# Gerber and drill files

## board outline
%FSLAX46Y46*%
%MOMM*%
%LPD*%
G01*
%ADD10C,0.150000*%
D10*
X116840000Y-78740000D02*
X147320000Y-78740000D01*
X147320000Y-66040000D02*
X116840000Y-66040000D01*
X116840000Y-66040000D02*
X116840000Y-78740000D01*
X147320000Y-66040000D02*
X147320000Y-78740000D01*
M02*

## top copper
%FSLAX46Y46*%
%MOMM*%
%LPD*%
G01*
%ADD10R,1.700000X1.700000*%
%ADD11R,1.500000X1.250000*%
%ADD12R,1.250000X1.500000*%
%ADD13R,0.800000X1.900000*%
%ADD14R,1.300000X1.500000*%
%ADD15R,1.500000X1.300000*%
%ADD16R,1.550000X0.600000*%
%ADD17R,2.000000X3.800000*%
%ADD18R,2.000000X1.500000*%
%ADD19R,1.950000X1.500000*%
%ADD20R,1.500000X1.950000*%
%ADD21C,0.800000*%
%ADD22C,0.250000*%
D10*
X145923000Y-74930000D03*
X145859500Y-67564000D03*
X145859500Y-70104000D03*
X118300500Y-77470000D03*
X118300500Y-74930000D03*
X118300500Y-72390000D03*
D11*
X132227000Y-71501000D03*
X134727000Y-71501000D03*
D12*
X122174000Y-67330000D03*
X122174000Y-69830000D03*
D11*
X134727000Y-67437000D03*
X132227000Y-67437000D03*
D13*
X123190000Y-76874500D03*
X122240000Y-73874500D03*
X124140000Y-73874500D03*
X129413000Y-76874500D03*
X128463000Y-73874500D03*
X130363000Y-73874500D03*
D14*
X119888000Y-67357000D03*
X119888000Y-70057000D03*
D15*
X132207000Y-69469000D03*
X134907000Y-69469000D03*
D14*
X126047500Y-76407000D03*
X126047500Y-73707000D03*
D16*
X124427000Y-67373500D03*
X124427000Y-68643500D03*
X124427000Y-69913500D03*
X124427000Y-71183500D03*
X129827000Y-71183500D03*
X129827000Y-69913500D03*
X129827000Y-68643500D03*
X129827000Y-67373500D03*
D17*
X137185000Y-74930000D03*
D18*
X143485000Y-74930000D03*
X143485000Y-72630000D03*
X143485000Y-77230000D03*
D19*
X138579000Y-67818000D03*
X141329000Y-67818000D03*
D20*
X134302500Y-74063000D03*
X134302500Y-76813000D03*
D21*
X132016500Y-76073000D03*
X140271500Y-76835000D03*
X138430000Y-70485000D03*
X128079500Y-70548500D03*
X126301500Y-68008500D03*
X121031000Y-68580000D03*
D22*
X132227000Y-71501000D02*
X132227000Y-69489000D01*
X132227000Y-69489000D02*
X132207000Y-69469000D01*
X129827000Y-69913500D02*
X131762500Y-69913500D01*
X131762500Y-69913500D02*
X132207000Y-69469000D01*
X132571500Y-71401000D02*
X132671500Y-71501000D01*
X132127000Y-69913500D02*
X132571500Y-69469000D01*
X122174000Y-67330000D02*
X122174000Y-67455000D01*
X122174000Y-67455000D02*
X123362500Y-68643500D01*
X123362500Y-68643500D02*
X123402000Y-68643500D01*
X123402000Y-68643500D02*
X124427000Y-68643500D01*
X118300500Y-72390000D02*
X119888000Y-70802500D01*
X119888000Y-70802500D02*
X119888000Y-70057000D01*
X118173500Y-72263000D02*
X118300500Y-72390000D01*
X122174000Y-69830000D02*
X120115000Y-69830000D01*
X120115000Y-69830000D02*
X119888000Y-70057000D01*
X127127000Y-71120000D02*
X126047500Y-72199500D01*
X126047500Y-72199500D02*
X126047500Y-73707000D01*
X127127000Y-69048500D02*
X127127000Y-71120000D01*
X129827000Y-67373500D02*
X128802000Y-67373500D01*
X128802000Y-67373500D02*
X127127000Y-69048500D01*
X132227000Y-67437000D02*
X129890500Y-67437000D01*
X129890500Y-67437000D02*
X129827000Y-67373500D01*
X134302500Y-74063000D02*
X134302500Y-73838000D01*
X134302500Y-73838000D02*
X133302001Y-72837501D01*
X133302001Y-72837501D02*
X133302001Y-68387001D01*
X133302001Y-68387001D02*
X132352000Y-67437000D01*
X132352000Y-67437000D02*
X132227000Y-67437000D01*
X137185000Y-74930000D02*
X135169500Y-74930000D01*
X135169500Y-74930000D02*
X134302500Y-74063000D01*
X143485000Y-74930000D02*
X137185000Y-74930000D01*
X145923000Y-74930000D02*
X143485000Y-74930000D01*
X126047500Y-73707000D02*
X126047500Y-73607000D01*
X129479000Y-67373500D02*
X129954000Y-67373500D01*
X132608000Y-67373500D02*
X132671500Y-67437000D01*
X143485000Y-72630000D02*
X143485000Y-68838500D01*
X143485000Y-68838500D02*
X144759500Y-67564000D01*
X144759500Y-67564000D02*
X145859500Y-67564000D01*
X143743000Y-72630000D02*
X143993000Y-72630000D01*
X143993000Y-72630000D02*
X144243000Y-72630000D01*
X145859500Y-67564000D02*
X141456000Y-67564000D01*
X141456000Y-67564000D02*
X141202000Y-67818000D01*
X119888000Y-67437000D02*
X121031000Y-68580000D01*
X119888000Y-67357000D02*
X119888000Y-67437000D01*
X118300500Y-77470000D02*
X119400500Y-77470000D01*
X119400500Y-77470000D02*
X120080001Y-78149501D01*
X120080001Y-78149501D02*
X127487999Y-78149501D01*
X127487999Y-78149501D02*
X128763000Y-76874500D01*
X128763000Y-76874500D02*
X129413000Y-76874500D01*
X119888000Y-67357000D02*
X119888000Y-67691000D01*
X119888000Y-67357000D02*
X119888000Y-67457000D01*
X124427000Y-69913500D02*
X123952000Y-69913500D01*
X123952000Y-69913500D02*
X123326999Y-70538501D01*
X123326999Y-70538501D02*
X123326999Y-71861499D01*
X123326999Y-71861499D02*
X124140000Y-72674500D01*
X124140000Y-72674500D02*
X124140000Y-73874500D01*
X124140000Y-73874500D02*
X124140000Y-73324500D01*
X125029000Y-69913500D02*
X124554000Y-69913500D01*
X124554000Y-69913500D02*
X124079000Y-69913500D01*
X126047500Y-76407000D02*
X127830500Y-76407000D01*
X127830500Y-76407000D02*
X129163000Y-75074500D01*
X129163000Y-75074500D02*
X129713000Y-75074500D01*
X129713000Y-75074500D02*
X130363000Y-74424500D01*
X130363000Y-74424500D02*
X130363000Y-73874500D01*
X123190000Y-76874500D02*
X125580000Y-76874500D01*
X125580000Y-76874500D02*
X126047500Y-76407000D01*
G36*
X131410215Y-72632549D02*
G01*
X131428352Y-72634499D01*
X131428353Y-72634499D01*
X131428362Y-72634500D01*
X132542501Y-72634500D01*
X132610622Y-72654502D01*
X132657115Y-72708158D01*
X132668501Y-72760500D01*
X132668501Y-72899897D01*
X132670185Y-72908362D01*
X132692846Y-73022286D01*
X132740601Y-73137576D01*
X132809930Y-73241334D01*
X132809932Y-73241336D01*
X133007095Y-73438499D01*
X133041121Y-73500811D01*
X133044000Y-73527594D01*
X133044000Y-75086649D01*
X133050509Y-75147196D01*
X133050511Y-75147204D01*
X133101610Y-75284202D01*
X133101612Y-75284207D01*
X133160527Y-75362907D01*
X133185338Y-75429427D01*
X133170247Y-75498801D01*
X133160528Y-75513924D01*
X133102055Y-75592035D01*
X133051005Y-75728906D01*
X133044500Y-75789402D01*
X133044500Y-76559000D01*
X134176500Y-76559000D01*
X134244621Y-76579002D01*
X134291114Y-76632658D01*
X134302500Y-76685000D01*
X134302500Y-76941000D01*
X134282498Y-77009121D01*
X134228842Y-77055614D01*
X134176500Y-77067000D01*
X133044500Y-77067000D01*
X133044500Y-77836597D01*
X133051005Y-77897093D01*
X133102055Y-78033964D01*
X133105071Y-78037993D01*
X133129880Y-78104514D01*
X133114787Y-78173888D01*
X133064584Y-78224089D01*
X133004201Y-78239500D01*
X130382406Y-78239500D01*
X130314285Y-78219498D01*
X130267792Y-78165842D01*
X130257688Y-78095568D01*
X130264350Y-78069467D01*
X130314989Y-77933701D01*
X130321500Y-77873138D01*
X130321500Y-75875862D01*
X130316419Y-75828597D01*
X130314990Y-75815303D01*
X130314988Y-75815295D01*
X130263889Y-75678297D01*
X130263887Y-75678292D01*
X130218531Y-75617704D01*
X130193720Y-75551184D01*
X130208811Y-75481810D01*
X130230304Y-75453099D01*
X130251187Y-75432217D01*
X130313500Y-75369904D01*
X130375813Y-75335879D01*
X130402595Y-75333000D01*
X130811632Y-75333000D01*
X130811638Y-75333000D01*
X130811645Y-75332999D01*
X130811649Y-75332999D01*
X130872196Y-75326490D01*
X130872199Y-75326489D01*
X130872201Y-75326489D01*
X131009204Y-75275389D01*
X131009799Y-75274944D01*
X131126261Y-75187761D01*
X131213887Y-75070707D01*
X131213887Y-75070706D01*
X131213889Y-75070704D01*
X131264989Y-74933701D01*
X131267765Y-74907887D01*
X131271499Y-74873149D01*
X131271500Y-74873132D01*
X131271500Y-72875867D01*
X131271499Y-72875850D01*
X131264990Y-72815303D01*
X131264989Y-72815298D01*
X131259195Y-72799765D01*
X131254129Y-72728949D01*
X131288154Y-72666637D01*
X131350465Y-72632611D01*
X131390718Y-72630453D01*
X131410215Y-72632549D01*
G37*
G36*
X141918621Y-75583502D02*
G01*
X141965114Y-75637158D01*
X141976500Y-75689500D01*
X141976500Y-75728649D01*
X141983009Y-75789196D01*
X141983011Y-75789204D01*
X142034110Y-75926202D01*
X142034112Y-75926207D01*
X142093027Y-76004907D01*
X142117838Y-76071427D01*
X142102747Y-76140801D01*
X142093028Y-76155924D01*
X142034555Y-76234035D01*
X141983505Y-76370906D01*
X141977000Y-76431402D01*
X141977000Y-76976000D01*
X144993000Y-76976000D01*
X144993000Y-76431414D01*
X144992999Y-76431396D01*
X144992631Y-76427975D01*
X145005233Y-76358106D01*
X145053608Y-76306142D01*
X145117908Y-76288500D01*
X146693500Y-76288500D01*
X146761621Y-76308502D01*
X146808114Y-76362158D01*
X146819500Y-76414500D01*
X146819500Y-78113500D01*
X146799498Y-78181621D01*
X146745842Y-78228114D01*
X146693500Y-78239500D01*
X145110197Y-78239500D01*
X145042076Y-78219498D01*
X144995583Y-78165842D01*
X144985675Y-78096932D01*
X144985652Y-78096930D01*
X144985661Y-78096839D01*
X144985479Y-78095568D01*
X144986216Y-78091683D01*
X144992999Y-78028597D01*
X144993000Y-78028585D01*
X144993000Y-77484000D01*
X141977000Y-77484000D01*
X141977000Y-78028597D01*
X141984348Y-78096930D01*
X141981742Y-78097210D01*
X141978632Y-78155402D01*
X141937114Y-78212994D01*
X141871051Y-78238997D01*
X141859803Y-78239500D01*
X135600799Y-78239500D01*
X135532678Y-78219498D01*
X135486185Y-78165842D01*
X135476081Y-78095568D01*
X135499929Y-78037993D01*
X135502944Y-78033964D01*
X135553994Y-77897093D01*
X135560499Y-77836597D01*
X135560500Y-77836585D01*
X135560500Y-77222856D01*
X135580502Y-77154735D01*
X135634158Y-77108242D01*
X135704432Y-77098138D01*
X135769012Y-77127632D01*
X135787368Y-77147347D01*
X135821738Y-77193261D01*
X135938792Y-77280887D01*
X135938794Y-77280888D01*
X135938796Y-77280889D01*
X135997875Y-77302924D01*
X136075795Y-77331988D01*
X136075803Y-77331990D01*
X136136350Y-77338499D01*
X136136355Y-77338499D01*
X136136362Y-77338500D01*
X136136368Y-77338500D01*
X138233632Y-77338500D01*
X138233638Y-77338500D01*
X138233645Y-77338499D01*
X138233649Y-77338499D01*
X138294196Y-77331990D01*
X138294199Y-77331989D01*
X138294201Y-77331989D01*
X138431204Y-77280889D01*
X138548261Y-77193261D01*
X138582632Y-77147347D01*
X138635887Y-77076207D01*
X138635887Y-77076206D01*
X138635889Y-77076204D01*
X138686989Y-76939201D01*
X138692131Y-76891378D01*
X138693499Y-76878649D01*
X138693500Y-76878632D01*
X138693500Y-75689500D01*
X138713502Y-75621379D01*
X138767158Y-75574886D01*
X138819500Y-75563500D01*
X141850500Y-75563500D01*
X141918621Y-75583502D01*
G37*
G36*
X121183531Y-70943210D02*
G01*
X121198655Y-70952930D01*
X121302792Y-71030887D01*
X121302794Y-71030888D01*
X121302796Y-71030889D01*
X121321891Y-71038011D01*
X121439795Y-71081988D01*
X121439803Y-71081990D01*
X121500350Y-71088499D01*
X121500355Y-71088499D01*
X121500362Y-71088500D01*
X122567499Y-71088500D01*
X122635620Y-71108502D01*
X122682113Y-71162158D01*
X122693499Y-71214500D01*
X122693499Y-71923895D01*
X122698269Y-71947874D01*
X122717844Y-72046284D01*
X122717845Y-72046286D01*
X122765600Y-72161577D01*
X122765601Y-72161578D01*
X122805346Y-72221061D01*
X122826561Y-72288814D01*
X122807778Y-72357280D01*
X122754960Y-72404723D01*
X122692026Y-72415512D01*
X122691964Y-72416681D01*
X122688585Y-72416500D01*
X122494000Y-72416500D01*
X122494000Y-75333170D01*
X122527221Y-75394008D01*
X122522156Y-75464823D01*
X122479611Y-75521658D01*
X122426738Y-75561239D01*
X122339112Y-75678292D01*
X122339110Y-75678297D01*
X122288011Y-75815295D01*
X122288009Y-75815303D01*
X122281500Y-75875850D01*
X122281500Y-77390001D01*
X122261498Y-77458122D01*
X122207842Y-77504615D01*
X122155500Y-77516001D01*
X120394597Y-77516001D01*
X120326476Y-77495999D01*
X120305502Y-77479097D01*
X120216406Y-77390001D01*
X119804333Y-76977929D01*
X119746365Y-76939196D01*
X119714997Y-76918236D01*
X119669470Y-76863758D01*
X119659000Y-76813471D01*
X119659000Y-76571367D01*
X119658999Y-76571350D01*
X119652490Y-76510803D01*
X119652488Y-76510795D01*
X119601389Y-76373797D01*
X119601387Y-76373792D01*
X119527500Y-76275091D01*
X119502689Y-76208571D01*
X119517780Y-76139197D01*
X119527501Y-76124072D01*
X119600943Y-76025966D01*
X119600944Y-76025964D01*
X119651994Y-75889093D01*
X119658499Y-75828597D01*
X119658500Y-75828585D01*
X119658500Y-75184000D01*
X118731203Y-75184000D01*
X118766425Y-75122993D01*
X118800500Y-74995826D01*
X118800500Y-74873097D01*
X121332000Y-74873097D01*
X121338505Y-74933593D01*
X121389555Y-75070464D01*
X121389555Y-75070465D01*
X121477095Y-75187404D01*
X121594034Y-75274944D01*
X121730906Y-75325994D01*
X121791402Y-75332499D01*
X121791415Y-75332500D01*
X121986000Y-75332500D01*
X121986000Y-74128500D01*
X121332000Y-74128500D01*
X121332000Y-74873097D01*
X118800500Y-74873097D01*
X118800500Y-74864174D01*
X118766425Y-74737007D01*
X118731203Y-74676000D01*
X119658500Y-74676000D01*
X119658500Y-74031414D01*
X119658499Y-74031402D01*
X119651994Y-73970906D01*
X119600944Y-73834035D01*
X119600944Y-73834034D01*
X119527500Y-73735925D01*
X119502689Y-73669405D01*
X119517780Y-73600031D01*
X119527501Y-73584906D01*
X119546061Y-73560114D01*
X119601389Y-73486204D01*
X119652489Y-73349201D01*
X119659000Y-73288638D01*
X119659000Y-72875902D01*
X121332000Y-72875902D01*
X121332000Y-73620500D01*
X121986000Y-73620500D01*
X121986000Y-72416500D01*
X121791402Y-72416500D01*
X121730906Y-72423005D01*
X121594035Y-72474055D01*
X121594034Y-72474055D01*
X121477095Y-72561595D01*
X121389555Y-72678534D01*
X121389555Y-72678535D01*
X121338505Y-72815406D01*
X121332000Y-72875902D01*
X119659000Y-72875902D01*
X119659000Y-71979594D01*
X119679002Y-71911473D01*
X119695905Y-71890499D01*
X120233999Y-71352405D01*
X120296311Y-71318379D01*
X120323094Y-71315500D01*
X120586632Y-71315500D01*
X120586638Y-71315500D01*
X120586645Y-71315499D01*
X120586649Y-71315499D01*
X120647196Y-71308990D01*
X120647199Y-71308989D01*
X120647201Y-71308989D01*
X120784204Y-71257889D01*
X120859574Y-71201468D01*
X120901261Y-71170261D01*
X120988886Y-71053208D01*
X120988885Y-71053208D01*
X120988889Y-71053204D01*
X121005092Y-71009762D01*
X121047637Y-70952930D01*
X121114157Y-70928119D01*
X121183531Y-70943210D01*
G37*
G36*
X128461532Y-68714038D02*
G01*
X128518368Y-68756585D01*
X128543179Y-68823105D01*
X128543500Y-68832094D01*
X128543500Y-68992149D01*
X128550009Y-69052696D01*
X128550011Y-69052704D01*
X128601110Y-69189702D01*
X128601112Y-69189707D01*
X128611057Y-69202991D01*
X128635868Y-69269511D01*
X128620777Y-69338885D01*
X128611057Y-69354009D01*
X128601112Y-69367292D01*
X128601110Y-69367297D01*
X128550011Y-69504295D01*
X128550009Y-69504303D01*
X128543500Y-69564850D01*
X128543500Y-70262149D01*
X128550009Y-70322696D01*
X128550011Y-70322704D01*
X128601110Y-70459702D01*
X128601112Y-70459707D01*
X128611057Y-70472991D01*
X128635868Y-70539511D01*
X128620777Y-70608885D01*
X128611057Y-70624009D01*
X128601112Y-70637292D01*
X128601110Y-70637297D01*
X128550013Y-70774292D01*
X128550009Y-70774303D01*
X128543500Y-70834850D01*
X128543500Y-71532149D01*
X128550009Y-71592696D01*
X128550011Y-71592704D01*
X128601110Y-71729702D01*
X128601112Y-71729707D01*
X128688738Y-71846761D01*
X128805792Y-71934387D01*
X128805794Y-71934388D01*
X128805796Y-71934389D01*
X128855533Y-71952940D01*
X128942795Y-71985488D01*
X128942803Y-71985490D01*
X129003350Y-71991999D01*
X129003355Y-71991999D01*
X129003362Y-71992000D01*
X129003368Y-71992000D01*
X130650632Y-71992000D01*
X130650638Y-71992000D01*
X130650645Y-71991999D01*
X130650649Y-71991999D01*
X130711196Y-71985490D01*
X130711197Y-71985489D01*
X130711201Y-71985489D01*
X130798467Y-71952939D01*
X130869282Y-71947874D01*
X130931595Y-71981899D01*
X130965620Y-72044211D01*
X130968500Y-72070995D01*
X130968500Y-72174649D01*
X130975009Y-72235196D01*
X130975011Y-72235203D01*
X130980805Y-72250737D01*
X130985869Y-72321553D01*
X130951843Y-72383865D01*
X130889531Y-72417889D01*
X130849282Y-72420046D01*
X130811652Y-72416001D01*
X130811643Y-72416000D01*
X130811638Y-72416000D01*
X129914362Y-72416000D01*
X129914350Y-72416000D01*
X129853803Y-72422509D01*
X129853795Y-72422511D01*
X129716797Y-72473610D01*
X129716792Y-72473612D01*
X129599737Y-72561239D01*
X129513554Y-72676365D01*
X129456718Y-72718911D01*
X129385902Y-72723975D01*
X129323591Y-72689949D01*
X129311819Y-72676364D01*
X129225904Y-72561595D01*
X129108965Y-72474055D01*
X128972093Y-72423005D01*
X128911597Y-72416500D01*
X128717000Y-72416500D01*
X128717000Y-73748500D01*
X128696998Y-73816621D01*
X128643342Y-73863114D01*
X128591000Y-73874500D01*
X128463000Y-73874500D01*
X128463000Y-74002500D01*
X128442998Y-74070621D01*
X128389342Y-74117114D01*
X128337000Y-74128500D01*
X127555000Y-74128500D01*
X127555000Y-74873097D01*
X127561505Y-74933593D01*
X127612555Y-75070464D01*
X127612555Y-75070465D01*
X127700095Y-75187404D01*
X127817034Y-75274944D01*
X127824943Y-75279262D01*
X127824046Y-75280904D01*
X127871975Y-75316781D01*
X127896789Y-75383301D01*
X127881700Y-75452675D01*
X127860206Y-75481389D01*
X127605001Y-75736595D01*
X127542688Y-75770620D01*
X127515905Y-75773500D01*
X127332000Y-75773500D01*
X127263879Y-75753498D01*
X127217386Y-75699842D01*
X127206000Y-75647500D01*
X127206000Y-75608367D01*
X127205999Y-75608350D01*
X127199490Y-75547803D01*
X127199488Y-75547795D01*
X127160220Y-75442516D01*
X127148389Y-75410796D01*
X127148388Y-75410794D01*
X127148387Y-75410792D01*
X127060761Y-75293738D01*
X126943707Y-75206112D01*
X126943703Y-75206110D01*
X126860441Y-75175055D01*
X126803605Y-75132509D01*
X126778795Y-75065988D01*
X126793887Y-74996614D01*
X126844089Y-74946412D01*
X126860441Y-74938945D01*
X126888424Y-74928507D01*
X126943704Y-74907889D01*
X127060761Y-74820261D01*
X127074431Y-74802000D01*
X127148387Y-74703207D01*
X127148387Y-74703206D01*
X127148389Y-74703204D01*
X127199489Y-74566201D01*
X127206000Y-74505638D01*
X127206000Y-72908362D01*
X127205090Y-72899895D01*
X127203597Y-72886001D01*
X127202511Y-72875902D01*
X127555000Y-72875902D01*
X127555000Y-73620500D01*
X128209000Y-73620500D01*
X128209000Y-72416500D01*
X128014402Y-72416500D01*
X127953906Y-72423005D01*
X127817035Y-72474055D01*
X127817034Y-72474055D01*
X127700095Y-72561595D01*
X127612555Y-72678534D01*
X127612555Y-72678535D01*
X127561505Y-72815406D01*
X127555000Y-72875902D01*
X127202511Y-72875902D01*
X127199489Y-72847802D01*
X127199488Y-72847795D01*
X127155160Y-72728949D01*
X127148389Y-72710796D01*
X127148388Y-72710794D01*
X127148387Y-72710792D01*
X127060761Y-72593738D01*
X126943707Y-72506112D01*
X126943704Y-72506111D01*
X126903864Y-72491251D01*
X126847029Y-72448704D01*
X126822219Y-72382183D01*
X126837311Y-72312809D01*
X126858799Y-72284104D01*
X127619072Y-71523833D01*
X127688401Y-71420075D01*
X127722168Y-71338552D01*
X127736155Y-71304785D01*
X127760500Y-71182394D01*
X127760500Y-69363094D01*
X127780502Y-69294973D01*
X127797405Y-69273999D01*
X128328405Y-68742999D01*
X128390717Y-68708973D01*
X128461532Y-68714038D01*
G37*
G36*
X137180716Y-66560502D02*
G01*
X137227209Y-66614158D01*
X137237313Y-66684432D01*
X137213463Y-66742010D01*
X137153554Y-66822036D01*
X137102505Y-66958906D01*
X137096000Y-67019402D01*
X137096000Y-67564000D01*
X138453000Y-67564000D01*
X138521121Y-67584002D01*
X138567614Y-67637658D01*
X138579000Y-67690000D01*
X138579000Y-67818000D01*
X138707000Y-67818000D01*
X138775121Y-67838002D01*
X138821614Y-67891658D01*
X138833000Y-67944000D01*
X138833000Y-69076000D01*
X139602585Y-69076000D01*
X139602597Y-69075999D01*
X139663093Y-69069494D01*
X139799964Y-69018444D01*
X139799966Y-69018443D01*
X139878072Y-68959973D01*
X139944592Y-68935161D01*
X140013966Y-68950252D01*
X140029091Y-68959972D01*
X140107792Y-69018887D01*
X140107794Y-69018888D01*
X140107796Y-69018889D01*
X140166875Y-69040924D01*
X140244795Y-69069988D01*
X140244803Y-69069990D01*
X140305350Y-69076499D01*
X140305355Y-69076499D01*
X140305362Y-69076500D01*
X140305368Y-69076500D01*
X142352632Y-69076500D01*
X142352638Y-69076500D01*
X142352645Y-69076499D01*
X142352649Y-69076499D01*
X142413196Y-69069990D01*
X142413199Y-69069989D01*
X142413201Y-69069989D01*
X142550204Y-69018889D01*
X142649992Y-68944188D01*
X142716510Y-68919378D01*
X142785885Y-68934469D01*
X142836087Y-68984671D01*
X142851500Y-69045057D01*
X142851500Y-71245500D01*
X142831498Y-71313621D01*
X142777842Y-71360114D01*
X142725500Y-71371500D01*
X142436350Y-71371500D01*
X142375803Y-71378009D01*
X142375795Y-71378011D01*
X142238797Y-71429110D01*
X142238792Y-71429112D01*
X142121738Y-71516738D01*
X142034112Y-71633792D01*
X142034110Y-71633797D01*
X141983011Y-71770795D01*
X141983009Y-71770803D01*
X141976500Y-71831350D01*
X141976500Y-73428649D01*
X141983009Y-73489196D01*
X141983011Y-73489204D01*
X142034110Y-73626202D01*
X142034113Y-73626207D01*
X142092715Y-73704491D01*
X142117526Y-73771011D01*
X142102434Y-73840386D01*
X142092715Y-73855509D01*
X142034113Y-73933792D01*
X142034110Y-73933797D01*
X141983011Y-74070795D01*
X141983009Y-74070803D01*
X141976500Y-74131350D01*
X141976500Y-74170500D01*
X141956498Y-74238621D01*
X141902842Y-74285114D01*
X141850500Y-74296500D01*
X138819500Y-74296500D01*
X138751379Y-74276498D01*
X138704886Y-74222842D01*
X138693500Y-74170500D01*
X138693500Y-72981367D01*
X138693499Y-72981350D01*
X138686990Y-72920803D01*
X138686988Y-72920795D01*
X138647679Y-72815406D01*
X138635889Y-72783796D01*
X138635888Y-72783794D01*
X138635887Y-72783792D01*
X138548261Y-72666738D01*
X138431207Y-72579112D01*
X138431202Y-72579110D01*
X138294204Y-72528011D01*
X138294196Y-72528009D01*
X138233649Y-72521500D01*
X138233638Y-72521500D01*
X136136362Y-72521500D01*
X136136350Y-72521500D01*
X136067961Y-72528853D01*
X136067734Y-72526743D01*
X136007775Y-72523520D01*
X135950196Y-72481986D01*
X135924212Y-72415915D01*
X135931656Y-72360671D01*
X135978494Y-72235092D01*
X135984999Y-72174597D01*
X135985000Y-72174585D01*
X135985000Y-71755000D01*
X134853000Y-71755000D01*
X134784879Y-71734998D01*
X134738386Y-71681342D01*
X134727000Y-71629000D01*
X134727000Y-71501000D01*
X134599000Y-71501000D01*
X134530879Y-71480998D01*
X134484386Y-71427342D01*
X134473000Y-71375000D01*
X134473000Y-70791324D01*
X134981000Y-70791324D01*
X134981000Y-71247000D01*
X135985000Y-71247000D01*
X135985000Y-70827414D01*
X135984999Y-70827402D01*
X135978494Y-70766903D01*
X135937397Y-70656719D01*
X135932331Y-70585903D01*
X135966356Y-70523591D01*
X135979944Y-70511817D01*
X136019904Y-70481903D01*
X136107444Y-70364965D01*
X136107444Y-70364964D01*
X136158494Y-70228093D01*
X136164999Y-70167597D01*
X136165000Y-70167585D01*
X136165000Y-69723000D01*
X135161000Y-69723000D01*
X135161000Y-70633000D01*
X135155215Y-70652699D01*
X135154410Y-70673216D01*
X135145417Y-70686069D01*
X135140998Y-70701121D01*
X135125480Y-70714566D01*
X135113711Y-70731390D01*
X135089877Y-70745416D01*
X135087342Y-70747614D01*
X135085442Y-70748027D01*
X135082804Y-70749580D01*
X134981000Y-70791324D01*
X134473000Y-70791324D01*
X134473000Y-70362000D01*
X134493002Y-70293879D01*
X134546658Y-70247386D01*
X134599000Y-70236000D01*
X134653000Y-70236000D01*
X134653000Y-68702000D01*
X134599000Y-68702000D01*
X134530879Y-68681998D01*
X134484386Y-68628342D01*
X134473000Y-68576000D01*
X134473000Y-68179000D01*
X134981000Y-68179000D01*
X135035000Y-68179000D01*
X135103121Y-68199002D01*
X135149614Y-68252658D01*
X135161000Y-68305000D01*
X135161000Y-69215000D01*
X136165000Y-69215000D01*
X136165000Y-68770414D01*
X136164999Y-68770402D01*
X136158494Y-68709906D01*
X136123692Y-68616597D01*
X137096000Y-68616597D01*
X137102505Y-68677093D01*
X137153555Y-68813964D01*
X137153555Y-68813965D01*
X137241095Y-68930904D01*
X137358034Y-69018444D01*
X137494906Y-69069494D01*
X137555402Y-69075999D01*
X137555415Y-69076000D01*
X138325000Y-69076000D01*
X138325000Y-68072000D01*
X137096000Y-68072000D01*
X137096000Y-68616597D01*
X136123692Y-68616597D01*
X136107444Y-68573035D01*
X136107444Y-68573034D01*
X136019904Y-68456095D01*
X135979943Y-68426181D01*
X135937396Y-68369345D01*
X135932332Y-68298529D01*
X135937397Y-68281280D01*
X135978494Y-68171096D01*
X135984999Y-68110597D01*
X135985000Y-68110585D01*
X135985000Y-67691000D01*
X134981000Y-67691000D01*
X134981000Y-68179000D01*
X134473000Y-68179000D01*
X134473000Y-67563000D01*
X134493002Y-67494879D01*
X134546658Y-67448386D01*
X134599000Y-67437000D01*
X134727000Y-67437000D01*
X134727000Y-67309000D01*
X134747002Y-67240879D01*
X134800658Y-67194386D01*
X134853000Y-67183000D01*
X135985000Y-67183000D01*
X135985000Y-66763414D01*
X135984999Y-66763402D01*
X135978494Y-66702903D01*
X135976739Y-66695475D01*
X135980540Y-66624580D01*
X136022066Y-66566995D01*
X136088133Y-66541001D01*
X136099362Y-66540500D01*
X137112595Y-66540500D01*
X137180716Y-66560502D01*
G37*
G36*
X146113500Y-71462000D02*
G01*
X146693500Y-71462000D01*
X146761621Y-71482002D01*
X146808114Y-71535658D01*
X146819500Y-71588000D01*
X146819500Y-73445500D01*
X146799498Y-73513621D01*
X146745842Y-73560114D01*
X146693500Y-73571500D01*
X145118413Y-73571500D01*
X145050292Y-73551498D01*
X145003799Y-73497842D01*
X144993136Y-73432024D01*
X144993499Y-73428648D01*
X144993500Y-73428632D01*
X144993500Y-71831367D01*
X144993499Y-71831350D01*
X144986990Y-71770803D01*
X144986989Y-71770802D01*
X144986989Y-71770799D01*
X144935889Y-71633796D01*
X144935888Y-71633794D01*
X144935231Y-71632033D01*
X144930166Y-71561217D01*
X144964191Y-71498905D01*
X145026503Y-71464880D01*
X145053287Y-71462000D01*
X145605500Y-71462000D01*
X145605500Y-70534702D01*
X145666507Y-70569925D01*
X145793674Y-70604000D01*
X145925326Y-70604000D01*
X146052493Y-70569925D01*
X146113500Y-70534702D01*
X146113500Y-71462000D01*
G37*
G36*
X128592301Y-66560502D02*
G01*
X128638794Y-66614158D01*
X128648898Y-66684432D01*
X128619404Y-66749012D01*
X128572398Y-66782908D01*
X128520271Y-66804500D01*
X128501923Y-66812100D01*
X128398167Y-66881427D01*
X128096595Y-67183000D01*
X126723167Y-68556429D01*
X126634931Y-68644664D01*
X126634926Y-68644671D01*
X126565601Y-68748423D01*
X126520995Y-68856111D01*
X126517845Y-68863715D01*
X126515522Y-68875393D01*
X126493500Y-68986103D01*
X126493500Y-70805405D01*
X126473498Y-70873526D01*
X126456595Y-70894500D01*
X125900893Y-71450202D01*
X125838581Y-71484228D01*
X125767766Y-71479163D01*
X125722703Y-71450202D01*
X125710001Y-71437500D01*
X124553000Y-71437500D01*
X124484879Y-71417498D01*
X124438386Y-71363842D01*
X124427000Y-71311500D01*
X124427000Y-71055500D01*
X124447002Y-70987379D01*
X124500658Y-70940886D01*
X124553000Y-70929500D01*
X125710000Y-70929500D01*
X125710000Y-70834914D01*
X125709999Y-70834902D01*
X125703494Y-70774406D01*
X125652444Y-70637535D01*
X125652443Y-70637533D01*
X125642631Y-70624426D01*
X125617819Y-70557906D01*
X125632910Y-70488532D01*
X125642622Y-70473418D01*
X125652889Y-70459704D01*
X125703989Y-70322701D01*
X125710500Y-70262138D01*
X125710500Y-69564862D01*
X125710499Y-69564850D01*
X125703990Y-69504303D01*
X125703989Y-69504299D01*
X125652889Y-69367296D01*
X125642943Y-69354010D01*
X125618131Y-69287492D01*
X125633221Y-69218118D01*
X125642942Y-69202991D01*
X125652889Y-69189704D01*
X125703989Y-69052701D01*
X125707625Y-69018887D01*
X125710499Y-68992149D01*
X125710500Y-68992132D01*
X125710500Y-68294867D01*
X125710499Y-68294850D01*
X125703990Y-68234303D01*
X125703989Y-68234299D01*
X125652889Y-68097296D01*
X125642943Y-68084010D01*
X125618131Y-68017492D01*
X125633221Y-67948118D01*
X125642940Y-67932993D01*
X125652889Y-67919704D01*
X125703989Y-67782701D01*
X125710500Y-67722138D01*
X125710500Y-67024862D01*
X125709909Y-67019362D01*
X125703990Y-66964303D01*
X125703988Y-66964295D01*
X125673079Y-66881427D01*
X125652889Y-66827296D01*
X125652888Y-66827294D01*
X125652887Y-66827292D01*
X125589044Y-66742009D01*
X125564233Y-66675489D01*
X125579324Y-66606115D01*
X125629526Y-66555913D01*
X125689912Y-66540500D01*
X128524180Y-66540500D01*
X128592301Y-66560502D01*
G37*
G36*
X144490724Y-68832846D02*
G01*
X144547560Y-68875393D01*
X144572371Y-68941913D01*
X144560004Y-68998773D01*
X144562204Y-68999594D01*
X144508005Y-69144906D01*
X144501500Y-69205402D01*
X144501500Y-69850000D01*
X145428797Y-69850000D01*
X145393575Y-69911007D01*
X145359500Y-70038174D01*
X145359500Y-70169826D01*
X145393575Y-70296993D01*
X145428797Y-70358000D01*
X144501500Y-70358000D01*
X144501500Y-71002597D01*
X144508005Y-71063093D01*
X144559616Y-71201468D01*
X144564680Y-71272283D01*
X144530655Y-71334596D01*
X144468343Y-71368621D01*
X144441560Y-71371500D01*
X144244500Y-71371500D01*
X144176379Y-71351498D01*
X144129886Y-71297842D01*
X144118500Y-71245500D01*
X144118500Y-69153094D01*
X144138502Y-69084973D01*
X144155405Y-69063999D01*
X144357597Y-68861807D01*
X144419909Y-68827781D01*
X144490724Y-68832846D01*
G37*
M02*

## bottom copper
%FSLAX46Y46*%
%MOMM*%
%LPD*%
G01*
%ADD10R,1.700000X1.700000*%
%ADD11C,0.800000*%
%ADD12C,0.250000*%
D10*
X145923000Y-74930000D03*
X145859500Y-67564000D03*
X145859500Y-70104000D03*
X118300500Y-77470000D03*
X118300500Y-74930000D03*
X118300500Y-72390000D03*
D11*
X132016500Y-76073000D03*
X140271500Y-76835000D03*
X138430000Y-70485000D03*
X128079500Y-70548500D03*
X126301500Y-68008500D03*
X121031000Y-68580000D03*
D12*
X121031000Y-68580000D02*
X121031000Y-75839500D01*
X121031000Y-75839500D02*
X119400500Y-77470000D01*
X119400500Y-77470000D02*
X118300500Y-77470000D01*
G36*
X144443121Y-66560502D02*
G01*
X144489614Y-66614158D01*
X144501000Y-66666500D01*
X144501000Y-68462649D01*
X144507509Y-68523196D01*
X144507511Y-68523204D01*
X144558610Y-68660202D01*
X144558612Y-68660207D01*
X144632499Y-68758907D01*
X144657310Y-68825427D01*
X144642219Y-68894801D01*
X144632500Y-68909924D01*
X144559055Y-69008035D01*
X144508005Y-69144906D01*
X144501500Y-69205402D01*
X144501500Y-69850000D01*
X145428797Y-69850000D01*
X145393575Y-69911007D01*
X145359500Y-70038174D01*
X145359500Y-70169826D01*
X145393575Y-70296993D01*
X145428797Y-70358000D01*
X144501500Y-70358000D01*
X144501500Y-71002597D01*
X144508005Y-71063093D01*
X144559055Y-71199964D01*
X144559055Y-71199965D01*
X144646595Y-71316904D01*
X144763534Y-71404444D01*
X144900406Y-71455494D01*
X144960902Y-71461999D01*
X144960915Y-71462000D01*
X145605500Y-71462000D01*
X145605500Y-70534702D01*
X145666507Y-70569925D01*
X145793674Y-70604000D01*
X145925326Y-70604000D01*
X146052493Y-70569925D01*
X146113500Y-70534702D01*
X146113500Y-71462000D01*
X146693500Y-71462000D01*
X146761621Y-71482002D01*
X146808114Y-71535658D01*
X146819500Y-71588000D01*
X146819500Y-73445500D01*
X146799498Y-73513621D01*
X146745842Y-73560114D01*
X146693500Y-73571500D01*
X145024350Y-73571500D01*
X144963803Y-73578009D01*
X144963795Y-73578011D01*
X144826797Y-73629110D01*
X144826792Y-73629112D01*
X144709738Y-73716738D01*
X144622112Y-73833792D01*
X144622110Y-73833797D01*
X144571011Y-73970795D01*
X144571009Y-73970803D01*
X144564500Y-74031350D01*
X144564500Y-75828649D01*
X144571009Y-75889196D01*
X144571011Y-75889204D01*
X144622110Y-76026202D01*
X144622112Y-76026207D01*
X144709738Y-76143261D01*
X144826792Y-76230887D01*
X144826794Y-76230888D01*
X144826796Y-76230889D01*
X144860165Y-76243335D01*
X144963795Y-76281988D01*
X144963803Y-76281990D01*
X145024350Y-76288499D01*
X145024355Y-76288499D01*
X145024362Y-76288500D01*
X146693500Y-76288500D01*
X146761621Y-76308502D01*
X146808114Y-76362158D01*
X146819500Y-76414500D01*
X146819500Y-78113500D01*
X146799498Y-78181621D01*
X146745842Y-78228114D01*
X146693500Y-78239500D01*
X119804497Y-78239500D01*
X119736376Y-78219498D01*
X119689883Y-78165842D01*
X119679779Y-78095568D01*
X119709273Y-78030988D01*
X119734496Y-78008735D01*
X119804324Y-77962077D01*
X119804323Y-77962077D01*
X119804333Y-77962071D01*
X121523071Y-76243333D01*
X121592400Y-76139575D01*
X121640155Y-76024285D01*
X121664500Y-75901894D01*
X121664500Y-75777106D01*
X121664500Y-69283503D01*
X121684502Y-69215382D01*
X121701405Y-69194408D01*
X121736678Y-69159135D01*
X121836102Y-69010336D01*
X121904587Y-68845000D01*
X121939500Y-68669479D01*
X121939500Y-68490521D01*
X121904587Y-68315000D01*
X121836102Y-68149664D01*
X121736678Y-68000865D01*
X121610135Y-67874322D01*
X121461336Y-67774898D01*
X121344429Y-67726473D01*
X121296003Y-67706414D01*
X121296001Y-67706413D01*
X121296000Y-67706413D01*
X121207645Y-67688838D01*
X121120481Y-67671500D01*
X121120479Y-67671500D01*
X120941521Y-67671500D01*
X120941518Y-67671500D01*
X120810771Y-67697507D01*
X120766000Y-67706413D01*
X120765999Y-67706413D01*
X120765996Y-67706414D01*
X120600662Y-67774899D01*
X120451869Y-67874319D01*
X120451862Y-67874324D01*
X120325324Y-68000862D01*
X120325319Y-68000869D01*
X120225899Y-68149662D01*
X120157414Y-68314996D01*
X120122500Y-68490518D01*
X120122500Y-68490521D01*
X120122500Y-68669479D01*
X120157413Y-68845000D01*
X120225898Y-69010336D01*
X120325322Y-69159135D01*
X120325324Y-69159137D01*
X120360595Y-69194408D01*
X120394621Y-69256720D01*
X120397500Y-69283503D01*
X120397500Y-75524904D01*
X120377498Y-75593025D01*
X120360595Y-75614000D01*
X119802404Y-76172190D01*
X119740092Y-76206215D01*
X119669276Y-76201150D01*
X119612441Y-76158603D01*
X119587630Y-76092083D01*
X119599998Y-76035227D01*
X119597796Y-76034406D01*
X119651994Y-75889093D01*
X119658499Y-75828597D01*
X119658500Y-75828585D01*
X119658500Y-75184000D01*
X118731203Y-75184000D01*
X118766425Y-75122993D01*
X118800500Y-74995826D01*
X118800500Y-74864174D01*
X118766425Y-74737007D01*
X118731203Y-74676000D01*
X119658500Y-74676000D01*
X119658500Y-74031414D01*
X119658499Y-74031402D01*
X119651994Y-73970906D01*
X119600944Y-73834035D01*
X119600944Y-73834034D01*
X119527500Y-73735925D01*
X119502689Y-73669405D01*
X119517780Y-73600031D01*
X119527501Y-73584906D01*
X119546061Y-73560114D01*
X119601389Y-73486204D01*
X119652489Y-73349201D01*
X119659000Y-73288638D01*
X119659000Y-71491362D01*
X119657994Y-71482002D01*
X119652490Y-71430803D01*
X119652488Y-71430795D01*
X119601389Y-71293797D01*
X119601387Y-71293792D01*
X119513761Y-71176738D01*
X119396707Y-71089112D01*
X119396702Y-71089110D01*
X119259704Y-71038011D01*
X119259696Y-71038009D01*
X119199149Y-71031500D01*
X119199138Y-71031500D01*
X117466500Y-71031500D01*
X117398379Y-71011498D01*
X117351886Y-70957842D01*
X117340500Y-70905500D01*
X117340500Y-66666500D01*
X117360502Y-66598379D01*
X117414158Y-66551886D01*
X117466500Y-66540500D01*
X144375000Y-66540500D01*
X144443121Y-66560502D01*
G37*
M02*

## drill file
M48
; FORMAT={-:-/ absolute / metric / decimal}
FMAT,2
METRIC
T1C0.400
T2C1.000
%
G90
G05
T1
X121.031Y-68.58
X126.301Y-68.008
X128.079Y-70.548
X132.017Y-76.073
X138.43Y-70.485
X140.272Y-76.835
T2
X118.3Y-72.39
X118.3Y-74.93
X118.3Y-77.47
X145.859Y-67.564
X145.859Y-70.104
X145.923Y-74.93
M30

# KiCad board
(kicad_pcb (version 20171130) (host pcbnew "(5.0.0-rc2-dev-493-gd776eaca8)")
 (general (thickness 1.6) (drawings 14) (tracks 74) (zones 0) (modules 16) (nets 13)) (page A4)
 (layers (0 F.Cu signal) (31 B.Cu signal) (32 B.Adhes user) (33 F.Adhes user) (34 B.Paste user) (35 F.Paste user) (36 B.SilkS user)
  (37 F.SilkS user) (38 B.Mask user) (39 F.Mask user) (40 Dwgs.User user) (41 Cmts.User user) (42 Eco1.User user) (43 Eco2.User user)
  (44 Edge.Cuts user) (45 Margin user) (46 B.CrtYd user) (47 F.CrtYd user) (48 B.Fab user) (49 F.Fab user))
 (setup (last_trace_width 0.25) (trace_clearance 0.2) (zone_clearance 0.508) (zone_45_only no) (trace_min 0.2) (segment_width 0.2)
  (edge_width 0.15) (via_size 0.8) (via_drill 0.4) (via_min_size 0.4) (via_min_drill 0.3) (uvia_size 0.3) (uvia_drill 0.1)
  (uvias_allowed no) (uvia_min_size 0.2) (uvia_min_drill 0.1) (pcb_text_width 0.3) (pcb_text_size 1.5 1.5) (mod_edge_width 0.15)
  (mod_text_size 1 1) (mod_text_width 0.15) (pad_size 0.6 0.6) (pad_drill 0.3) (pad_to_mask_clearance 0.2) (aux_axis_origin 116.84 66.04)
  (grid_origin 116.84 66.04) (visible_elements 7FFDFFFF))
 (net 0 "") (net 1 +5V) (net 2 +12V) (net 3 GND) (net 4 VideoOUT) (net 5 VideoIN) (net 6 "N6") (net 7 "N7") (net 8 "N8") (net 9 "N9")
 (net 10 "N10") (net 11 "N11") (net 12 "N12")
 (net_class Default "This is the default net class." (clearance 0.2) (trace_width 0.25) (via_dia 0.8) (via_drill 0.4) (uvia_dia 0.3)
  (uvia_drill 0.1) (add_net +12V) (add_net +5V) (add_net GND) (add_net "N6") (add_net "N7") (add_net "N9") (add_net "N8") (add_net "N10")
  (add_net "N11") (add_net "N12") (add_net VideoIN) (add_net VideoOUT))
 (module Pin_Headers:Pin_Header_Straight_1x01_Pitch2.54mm (layer F.Cu) (at 145.923 74.93)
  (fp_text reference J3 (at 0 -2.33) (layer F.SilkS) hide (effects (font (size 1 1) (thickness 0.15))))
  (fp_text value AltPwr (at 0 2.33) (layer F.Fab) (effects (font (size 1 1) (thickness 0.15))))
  (pad 1 thru_hole rect (at 0 0) (size 1.7 1.7) (drill 1) (layers *.Cu *.Mask) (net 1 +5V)))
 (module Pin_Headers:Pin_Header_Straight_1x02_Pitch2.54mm (layer F.Cu) (at 145.8595 67.564)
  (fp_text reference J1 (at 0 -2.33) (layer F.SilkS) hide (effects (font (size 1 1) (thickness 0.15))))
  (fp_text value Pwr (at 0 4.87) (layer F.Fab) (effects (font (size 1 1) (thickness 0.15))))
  (pad 1 thru_hole rect (at 0 0) (size 1.7 1.7) (drill 1) (layers *.Cu *.Mask) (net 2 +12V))
  (pad 2 thru_hole rect (at 0 2.54) (size 1.7 1.7) (drill 1) (layers *.Cu *.Mask) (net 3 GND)))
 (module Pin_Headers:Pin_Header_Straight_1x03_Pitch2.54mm (layer F.Cu) (at 118.3005 77.47 180)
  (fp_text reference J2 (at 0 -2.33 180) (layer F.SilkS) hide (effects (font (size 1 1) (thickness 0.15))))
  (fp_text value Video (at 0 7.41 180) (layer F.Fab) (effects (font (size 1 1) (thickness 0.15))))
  (pad 1 thru_hole rect (at 0 0 180) (size 1.7 1.7) (drill 1) (layers *.Cu *.Mask) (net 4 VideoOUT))
  (pad 2 thru_hole rect (at 0 2.54 180) (size 1.7 1.7) (drill 1) (layers *.Cu *.Mask) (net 3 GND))
  (pad 3 thru_hole rect (at 0 5.08 180) (size 1.7 1.7) (drill 1) (layers *.Cu *.Mask) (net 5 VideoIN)))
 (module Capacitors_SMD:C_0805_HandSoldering (layer F.Cu) (at 133.477 71.501)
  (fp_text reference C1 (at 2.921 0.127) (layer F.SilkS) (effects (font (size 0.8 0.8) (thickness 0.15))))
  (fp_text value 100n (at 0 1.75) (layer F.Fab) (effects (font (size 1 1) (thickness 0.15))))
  (pad 1 smd rect (at -1.25 0) (size 1.5 1.25) (layers F.Cu F.Paste F.Mask) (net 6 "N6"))
  (pad 2 smd rect (at 1.25 0) (size 1.5 1.25) (layers F.Cu F.Paste F.Mask) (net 3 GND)))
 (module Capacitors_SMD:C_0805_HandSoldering (layer F.Cu) (at 122.174 68.58 90)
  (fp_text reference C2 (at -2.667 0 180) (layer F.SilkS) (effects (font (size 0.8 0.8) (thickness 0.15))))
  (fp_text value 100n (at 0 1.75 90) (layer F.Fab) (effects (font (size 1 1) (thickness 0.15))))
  (pad 2 smd rect (at 1.25 0 90) (size 1.5 1.25) (layers F.Cu F.Paste F.Mask) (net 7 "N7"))
  (pad 1 smd rect (at -1.25 0 90) (size 1.5 1.25) (layers F.Cu F.Paste F.Mask) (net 5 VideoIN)))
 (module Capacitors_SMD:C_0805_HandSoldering (layer F.Cu) (at 133.477 67.437 180)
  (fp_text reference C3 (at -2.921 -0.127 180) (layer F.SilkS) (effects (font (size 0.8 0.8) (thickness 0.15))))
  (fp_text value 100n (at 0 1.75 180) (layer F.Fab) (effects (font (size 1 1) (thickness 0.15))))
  (pad 1 smd rect (at -1.25 0 180) (size 1.5 1.25) (layers F.Cu F.Paste F.Mask) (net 3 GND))
  (pad 2 smd rect (at 1.25 0 180) (size 1.5 1.25) (layers F.Cu F.Paste F.Mask) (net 1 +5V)))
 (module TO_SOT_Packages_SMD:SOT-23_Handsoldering (layer F.Cu) (at 123.19 75.3745 270)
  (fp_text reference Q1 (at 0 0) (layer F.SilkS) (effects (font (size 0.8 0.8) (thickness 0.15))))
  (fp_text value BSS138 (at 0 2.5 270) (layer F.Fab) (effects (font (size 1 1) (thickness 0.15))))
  (pad 3 smd rect (at 1.5 0 270) (size 1.9 0.8) (layers F.Cu F.Paste F.Mask) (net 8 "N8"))
  (pad 2 smd rect (at -1.5 0.95 270) (size 1.9 0.8) (layers F.Cu F.Paste F.Mask) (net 3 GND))
  (pad 1 smd rect (at -1.5 -0.95 270) (size 1.9 0.8) (layers F.Cu F.Paste F.Mask) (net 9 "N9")))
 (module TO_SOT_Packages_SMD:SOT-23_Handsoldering (layer F.Cu) (at 129.413 75.3745 270)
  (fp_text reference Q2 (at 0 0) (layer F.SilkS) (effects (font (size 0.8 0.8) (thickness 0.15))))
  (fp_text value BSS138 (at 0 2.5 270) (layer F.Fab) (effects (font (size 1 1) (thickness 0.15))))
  (pad 3 smd rect (at 1.5 0 270) (size 1.9 0.8) (layers F.Cu F.Paste F.Mask) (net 4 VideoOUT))
  (pad 2 smd rect (at -1.5 0.95 270) (size 1.9 0.8) (layers F.Cu F.Paste F.Mask) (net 3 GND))
  (pad 1 smd rect (at -1.5 -0.95 270) (size 1.9 0.8) (layers F.Cu F.Paste F.Mask) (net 8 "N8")))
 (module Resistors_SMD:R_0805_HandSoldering (layer F.Cu) (at 119.888 68.707 90)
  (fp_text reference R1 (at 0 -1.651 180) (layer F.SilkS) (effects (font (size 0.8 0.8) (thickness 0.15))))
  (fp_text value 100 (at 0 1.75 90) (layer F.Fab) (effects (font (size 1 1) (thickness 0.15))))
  (pad 2 smd rect (at 1.35 0 90) (size 1.5 1.3) (layers F.Cu F.Paste F.Mask) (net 4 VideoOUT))
  (pad 1 smd rect (at -1.35 0 90) (size 1.5 1.3) (layers F.Cu F.Paste F.Mask) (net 5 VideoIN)))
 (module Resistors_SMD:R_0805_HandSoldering (layer F.Cu) (at 133.557 69.469)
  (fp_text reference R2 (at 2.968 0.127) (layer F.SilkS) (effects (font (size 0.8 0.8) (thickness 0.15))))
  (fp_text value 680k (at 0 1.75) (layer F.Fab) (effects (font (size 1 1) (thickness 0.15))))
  (pad 1 smd rect (at -1.35 0) (size 1.5 1.3) (layers F.Cu F.Paste F.Mask) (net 6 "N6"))
  (pad 2 smd rect (at 1.35 0) (size 1.5 1.3) (layers F.Cu F.Paste F.Mask) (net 3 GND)))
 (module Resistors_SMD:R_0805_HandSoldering (layer F.Cu) (at 126.0475 75.057 270)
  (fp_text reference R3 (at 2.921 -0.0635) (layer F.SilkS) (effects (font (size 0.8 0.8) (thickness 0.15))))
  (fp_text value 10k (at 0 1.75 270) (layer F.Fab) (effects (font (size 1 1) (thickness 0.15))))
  (pad 2 smd rect (at 1.35 0 270) (size 1.5 1.3) (layers F.Cu F.Paste F.Mask) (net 8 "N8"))
  (pad 1 smd rect (at -1.35 0 270) (size 1.5 1.3) (layers F.Cu F.Paste F.Mask) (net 1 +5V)))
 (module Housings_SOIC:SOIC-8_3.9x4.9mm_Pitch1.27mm (layer F.Cu) (at 127.127 69.2785)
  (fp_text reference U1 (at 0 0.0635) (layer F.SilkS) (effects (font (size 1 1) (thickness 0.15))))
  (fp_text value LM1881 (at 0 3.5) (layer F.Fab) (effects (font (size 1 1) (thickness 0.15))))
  (pad 1 smd rect (at -2.7 -1.905) (size 1.55 0.6) (layers F.Cu F.Paste F.Mask) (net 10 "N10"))
  (pad 2 smd rect (at -2.7 -0.635) (size 1.55 0.6) (layers F.Cu F.Paste F.Mask) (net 7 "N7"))
  (pad 3 smd rect (at -2.7 0.635) (size 1.55 0.6) (layers F.Cu F.Paste F.Mask) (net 9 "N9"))
  (pad 4 smd rect (at -2.7 1.905) (size 1.55 0.6) (layers F.Cu F.Paste F.Mask) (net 3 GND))
  (pad 5 smd rect (at 2.7 1.905) (size 1.55 0.6) (layers F.Cu F.Paste F.Mask) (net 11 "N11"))
  (pad 6 smd rect (at 2.7 0.635) (size 1.55 0.6) (layers F.Cu F.Paste F.Mask) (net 6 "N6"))
  (pad 7 smd rect (at 2.7 -0.635) (size 1.55 0.6) (layers F.Cu F.Paste F.Mask) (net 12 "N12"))
  (pad 8 smd rect (at 2.7 -1.905) (size 1.55 0.6) (layers F.Cu F.Paste F.Mask) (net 1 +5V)))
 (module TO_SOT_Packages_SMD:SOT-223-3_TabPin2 (layer F.Cu) (at 140.335 74.93 180)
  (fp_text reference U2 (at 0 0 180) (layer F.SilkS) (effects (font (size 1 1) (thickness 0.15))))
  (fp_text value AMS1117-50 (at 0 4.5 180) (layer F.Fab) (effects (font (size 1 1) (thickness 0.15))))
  (pad 2 smd rect (at 3.15 0 180) (size 2 3.8) (layers F.Cu F.Paste F.Mask) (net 1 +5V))
  (pad 2 smd rect (at -3.15 0 180) (size 2 1.5) (layers F.Cu F.Paste F.Mask) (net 1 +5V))
  (pad 3 smd rect (at -3.15 2.3 180) (size 2 1.5) (layers F.Cu F.Paste F.Mask) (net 2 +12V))
  (pad 1 smd rect (at -3.15 -2.3 180) (size 2 1.5) (layers F.Cu F.Paste F.Mask) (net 3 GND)))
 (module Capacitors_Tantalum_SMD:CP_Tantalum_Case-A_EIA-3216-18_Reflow (layer F.Cu) (at 139.954 67.818 180)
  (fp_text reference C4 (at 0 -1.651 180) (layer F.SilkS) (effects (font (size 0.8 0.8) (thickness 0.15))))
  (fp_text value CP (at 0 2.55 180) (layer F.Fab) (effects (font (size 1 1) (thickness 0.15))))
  (pad 2 smd rect (at 1.375 0 180) (size 1.95 1.5) (layers F.Cu F.Paste F.Mask) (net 3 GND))
  (pad 1 smd rect (at -1.375 0 180) (size 1.95 1.5) (layers F.Cu F.Paste F.Mask) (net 2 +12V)))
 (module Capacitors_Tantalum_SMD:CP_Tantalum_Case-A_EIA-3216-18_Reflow (layer F.Cu) (at 134.3025 75.438 270)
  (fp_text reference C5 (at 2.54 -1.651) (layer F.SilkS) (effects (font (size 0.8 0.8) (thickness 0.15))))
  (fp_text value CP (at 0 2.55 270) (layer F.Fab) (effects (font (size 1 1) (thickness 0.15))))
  (pad 1 smd rect (at -1.375 0 270) (size 1.95 1.5) (layers F.Cu F.Paste F.Mask) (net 1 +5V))
  (pad 2 smd rect (at 1.375 0 270) (size 1.95 1.5) (layers F.Cu F.Paste F.Mask) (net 3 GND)))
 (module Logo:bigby (layer B.Cu) (at 124.714 70.612 180)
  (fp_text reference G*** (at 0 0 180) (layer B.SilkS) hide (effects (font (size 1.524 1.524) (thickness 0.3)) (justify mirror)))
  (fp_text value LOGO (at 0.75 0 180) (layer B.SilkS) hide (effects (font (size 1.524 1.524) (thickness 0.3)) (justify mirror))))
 (gr_line (start 116.84 78.74) (end 147.32 78.74) (angle 90) (layer Edge.Cuts) (width 0.15))
 (gr_line (start 147.32 66.04) (end 116.84 66.04) (angle 90) (layer Edge.Cuts) (width 0.15))
 (gr_line (start 116.84 66.04) (end 116.84 78.74) (angle 90) (layer Edge.Cuts) (width 0.15))
 (gr_line (start 147.32 66.04) (end 147.32 78.74) (angle 90) (layer Edge.Cuts) (width 0.15))
 (segment (start 132.227 71.501) (end 132.227 69.489) (width 0.25) (layer F.Cu) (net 6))
 (segment (start 132.227 69.489) (end 132.207 69.469) (width 0.25) (layer F.Cu) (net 6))
 (segment (start 129.827 69.9135) (end 131.7625 69.9135) (width 0.25) (layer F.Cu) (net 6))
 (segment (start 131.7625 69.9135) (end 132.207 69.469) (width 0.25) (layer F.Cu) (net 6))
 (segment (start 132.5715 71.401) (end 132.6715 71.501) (width 0.25) (layer F.Cu) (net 6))
 (segment (start 132.127 69.9135) (end 132.5715 69.469) (width 0.25) (layer F.Cu) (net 6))
 (via (at 132.0165 76.073) (size 0.8) (drill 0.4) (layers F.Cu B.Cu) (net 3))
 (via (at 140.2715 76.835) (size 0.8) (drill 0.4) (layers F.Cu B.Cu) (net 3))
 (via (at 138.43 70.485) (size 0.8) (drill 0.4) (layers F.Cu B.Cu) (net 3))
 (via (at 128.0795 70.5485) (size 0.8) (drill 0.4) (layers F.Cu B.Cu) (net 3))
 (via (at 126.3015 68.0085) (size 0.8) (drill 0.4) (layers F.Cu B.Cu) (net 3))
 (segment (start 122.174 67.33) (end 122.174 67.455) (width 0.25) (layer F.Cu) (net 7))
 (segment (start 122.174 67.455) (end 123.3625 68.6435) (width 0.25) (layer F.Cu) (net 7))
 (segment (start 123.3625 68.6435) (end 123.402 68.6435) (width 0.25) (layer F.Cu) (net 7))
 (segment (start 123.402 68.6435) (end 124.427 68.6435) (width 0.25) (layer F.Cu) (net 7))
 (segment (start 118.3005 72.39) (end 119.888 70.8025) (width 0.25) (layer F.Cu) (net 5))
 (segment (start 119.888 70.8025) (end 119.888 70.057) (width 0.25) (layer F.Cu) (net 5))
 (segment (start 118.1735 72.263) (end 118.3005 72.39) (width 0.25) (layer F.Cu) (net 5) (status 30))
 (segment (start 122.174 69.83) (end 120.115 69.83) (width 0.25) (layer F.Cu) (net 5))
 (segment (start 120.115 69.83) (end 119.888 70.057) (width 0.25) (layer F.Cu) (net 5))
 (segment (start 127.127 71.12) (end 126.0475 72.1995) (width 0.25) (layer F.Cu) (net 1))
 (segment (start 126.0475 72.1995) (end 126.0475 73.707) (width 0.25) (layer F.Cu) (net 1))
 (segment (start 127.127 69.0485) (end 127.127 71.12) (width 0.25) (layer F.Cu) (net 1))
 (segment (start 129.827 67.3735) (end 128.802 67.3735) (width 0.25) (layer F.Cu) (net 1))
 (segment (start 128.802 67.3735) (end 127.127 69.0485) (width 0.25) (layer F.Cu) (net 1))
 (segment (start 132.227 67.437) (end 129.8905 67.437) (width 0.25) (layer F.Cu) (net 1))
 (segment (start 129.8905 67.437) (end 129.827 67.3735) (width 0.25) (layer F.Cu) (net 1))
 (segment (start 134.3025 74.063) (end 134.3025 73.838) (width 0.25) (layer F.Cu) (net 1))
 (segment (start 134.3025 73.838) (end 133.302001 72.837501) (width 0.25) (layer F.Cu) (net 1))
 (segment (start 133.302001 72.837501) (end 133.302001 68.387001) (width 0.25) (layer F.Cu) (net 1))
 (segment (start 133.302001 68.387001) (end 132.352 67.437) (width 0.25) (layer F.Cu) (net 1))
 (segment (start 132.352 67.437) (end 132.227 67.437) (width 0.25) (layer F.Cu) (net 1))
 (segment (start 137.185 74.93) (end 135.1695 74.93) (width 0.25) (layer F.Cu) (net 1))
 (segment (start 135.1695 74.93) (end 134.3025 74.063) (width 0.25) (layer F.Cu) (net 1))
 (segment (start 143.485 74.93) (end 137.185 74.93) (width 0.25) (layer F.Cu) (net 1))
 (segment (start 145.923 74.93) (end 143.485 74.93) (width 0.25) (layer F.Cu) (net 1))
 (segment (start 126.0475 73.707) (end 126.0475 73.607) (width 0.25) (layer F.Cu) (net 1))
 (segment (start 129.479 67.3735) (end 129.954 67.3735) (width 0.25) (layer F.Cu) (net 1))
 (segment (start 132.608 67.3735) (end 132.6715 67.437) (width 0.25) (layer F.Cu) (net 1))
 (segment (start 143.485 72.63) (end 143.485 68.8385) (width 0.25) (layer F.Cu) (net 2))
 (segment (start 143.485 68.8385) (end 144.7595 67.564) (width 0.25) (layer F.Cu) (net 2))
 (segment (start 144.7595 67.564) (end 145.8595 67.564) (width 0.25) (layer F.Cu) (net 2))
 (segment (start 143.743 72.63) (end 143.993 72.63) (width 0.25) (layer F.Cu) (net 2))
 (segment (start 143.993 72.63) (end 144.243 72.63) (width 0.25) (layer F.Cu) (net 2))
 (segment (start 145.8595 67.564) (end 141.456 67.564) (width 0.25) (layer F.Cu) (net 2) (status 10))
 (segment (start 141.456 67.564) (end 141.202 67.818) (width 0.25) (layer F.Cu) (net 2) (status 30))
 (segment (start 121.031 68.58) (end 121.031 75.8395) (width 0.25) (layer B.Cu) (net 4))
 (segment (start 121.031 75.8395) (end 119.4005 77.47) (width 0.25) (layer B.Cu) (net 4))
 (segment (start 119.4005 77.47) (end 118.3005 77.47) (width 0.25) (layer B.Cu) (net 4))
 (segment (start 119.888 67.437) (end 121.031 68.58) (width 0.25) (layer F.Cu) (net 4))
 (segment (start 119.888 67.357) (end 119.888 67.437) (width 0.25) (layer F.Cu) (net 4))
 (via (at 121.031 68.58) (size 0.8) (drill 0.4) (layers F.Cu B.Cu) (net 4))
 (segment (start 118.3005 77.47) (end 119.4005 77.47) (width 0.25) (layer F.Cu) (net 4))
 (segment (start 119.4005 77.47) (end 120.080001 78.149501) (width 0.25) (layer F.Cu) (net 4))
 (segment (start 120.080001 78.149501) (end 127.487999 78.149501) (width 0.25) (layer F.Cu) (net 4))
 (segment (start 127.487999 78.149501) (end 128.763 76.8745) (width 0.25) (layer F.Cu) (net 4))
 (segment (start 128.763 76.8745) (end 129.413 76.8745) (width 0.25) (layer F.Cu) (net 4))
 (segment (start 119.888 67.357) (end 119.888 67.691) (width 0.25) (layer F.Cu) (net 4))
 (segment (start 119.888 67.357) (end 119.888 67.457) (width 0.25) (layer F.Cu) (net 4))
 (segment (start 124.427 69.9135) (end 123.952 69.9135) (width 0.25) (layer F.Cu) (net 9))
 (segment (start 123.952 69.9135) (end 123.326999 70.538501) (width 0.25) (layer F.Cu) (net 9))
 (segment (start 123.326999 70.538501) (end 123.326999 71.861499) (width 0.25) (layer F.Cu) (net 9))
 (segment (start 123.326999 71.861499) (end 124.14 72.6745) (width 0.25) (layer F.Cu) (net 9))
 (segment (start 124.14 72.6745) (end 124.14 73.8745) (width 0.25) (layer F.Cu) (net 9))
 (segment (start 124.14 73.8745) (end 124.14 73.3245) (width 0.25) (layer F.Cu) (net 9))
 (segment (start 125.029 69.9135) (end 124.554 69.9135) (width 0.25) (layer F.Cu) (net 9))
 (segment (start 124.554 69.9135) (end 124.079 69.9135) (width 0.25) (layer F.Cu) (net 9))
 (segment (start 126.0475 76.407) (end 127.8305 76.407) (width 0.25) (layer F.Cu) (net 8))
 (segment (start 127.8305 76.407) (end 129.163 75.0745) (width 0.25) (layer F.Cu) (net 8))
 (segment (start 129.163 75.0745) (end 129.713 75.0745) (width 0.25) (layer F.Cu) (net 8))
 (segment (start 129.713 75.0745) (end 130.363 74.4245) (width 0.25) (layer F.Cu) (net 8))
 (segment (start 130.363 74.4245) (end 130.363 73.8745) (width 0.25) (layer F.Cu) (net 8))
 (segment (start 123.19 76.8745) (end 125.58 76.8745) (width 0.25) (layer F.Cu) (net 8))
 (segment (start 125.58 76.8745) (end 126.0475 76.407) (width 0.25) (layer F.Cu) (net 8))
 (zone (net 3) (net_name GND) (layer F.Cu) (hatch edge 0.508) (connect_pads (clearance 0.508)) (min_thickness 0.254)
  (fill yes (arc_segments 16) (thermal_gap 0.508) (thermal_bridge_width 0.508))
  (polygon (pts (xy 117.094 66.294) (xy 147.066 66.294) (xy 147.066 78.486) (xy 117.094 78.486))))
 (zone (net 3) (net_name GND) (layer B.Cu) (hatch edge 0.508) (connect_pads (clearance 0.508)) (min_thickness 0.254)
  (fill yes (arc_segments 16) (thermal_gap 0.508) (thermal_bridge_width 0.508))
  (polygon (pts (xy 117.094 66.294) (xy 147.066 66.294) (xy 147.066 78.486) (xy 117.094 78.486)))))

